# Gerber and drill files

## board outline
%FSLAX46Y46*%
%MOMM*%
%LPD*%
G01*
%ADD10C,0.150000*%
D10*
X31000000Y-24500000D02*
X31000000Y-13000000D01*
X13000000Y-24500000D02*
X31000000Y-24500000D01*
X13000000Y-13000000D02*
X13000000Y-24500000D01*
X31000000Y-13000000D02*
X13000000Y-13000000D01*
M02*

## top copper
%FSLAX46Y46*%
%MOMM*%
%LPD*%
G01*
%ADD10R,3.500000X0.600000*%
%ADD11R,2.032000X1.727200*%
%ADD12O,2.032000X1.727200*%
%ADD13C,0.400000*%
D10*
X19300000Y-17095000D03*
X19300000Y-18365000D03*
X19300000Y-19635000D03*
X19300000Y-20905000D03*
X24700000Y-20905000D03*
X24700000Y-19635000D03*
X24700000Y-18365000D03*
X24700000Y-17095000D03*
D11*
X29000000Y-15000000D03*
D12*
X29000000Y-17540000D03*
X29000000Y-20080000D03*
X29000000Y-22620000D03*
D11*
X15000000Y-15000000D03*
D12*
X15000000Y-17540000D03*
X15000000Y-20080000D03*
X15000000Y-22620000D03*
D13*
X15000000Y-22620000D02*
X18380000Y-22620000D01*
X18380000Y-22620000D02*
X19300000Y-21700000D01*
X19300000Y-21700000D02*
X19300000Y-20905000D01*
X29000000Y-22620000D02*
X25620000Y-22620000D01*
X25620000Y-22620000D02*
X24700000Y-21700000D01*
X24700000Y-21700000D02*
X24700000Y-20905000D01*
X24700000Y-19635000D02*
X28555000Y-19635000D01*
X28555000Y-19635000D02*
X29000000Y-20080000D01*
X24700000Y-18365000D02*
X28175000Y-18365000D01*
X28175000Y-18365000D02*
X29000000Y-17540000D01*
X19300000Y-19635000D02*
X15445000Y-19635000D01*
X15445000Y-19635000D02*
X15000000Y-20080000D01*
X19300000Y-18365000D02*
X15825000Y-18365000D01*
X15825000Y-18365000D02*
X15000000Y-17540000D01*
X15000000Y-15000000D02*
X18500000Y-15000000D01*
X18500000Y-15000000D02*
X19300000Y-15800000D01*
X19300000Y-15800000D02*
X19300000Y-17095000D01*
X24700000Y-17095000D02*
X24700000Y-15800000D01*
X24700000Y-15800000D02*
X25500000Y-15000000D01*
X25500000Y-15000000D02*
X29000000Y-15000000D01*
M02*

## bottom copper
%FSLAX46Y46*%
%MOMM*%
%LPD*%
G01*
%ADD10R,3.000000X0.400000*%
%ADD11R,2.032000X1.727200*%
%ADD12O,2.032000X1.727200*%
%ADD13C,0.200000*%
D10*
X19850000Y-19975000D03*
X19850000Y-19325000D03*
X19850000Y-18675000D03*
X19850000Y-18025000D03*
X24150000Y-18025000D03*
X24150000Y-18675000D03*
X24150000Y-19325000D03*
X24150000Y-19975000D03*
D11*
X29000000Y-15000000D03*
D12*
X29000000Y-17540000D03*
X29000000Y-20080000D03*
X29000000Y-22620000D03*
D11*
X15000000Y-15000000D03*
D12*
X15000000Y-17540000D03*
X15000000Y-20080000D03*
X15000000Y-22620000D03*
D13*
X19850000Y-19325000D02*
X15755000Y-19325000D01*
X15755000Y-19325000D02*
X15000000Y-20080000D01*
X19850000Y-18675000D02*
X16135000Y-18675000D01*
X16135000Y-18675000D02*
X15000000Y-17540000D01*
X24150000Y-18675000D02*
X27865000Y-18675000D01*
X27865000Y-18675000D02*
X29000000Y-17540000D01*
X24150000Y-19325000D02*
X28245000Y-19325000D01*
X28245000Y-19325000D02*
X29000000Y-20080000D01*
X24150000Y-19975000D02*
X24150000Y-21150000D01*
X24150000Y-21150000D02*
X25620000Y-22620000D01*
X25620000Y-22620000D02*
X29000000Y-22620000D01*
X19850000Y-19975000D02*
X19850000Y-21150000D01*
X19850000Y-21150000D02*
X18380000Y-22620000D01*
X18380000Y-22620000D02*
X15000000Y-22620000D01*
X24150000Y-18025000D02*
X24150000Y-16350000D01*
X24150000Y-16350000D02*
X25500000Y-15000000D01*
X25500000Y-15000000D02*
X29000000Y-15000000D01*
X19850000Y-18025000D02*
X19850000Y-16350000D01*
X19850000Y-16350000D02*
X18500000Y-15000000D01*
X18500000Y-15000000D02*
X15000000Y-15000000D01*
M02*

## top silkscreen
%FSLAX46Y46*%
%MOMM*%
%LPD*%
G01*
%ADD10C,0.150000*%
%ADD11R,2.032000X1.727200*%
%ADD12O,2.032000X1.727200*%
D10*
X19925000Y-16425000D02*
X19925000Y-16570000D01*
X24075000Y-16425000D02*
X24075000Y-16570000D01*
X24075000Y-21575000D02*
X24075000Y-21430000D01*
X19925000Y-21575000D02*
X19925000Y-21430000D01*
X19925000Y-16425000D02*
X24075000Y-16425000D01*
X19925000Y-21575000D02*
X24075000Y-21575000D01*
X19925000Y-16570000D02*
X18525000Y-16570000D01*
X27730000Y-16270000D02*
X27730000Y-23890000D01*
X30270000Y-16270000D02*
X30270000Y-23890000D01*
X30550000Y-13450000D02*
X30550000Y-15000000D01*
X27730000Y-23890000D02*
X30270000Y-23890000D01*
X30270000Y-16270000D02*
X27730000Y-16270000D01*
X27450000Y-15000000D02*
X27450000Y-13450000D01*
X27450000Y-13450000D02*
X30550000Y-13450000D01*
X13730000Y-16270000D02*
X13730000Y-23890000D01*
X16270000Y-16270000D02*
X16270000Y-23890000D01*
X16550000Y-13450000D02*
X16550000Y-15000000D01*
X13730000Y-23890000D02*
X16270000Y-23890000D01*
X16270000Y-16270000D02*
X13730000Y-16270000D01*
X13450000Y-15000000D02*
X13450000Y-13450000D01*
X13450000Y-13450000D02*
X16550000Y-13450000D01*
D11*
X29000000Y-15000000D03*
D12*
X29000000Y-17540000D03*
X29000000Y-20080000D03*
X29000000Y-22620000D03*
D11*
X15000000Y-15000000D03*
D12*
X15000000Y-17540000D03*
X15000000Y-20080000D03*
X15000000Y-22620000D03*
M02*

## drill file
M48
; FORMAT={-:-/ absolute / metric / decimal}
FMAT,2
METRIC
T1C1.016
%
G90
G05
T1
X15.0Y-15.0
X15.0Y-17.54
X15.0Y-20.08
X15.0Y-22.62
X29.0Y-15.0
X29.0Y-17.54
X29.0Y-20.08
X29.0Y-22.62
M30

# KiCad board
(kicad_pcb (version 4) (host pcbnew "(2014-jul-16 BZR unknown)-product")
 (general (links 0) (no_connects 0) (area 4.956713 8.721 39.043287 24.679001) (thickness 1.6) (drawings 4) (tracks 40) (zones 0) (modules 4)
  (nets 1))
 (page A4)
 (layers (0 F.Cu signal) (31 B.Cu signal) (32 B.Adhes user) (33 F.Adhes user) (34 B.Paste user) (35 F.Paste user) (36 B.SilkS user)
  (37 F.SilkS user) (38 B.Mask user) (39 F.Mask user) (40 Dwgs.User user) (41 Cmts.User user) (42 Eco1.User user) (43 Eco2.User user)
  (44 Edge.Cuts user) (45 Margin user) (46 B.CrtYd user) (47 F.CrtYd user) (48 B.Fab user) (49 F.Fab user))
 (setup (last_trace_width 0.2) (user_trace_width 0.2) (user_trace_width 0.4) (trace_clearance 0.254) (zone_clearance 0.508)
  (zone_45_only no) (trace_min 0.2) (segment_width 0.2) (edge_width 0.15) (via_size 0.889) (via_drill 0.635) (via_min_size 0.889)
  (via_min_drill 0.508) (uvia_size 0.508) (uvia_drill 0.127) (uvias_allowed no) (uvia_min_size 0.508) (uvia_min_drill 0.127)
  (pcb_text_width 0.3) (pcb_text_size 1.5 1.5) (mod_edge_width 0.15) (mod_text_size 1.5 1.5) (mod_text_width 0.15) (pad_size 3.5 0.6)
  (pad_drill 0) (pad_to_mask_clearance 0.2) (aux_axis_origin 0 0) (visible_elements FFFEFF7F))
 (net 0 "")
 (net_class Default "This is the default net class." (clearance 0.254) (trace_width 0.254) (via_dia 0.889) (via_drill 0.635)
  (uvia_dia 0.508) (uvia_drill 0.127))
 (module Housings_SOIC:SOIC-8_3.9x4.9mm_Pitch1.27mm (layer F.Cu) (at 22 19)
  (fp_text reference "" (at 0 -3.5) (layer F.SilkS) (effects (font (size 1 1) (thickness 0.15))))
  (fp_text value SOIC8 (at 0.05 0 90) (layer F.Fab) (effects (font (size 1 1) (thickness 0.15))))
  (fp_line (start -2.075 -2.575) (end -2.075 -2.43) (layer F.SilkS) (width 0.15))
  (fp_line (start 2.075 -2.575) (end 2.075 -2.43) (layer F.SilkS) (width 0.15))
  (fp_line (start 2.075 2.575) (end 2.075 2.43) (layer F.SilkS) (width 0.15))
  (fp_line (start -2.075 2.575) (end -2.075 2.43) (layer F.SilkS) (width 0.15))
  (fp_line (start -2.075 -2.575) (end 2.075 -2.575) (layer F.SilkS) (width 0.15))
  (fp_line (start -2.075 2.575) (end 2.075 2.575) (layer F.SilkS) (width 0.15))
  (fp_line (start -2.075 -2.43) (end -3.475 -2.43) (layer F.SilkS) (width 0.15))
  (pad 1 smd rect (at -2.7 -1.905) (size 3.5 0.6) (layers F.Cu F.Paste F.Mask))
  (pad 2 smd rect (at -2.7 -0.635) (size 3.5 0.6) (layers F.Cu F.Paste F.Mask))
  (pad 3 smd rect (at -2.7 0.635) (size 3.5 0.6) (layers F.Cu F.Paste F.Mask))
  (pad 4 smd rect (at -2.7 1.905) (size 3.5 0.6) (layers F.Cu F.Paste F.Mask))
  (pad 5 smd rect (at 2.7 1.905) (size 3.5 0.6) (layers F.Cu F.Paste F.Mask))
  (pad 6 smd rect (at 2.7 0.635) (size 3.5 0.6) (layers F.Cu F.Paste F.Mask))
  (pad 7 smd rect (at 2.7 -0.635) (size 3.5 0.6) (layers F.Cu F.Paste F.Mask))
  (pad 8 smd rect (at 2.7 -1.905) (size 3.5 0.6) (layers F.Cu F.Paste F.Mask)))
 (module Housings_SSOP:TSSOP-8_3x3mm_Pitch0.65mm (layer B.Cu) (at 22 19)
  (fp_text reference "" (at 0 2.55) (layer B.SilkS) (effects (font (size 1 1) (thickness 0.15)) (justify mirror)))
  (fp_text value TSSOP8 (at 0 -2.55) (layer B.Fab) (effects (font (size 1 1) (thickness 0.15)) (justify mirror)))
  (pad 1 smd rect (at -2.15 0.975) (size 3 0.4) (layers B.Cu B.Paste B.Mask))
  (pad 2 smd rect (at -2.15 0.325) (size 3 0.4) (layers B.Cu B.Paste B.Mask))
  (pad 3 smd rect (at -2.15 -0.325) (size 3 0.4) (layers B.Cu B.Paste B.Mask))
  (pad 4 smd rect (at -2.15 -0.975) (size 3 0.4) (layers B.Cu B.Paste B.Mask))
  (pad 5 smd rect (at 2.15 -0.975) (size 3 0.4) (layers B.Cu B.Paste B.Mask))
  (pad 6 smd rect (at 2.15 -0.325) (size 3 0.4) (layers B.Cu B.Paste B.Mask))
  (pad 7 smd rect (at 2.15 0.325) (size 3 0.4) (layers B.Cu B.Paste B.Mask))
  (pad 8 smd rect (at 2.15 0.975) (size 3 0.4) (layers B.Cu B.Paste B.Mask)))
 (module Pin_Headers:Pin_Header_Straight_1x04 (layer F.Cu) (at 29 15)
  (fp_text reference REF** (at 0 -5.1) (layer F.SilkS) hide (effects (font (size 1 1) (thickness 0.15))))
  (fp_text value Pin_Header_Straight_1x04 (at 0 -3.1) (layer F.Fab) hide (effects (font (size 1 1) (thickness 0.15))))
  (fp_line (start -1.27 1.27) (end -1.27 8.89) (layer F.SilkS) (width 0.15))
  (fp_line (start 1.27 1.27) (end 1.27 8.89) (layer F.SilkS) (width 0.15))
  (fp_line (start 1.55 -1.55) (end 1.55 0) (layer F.SilkS) (width 0.15))
  (fp_line (start -1.27 8.89) (end 1.27 8.89) (layer F.SilkS) (width 0.15))
  (fp_line (start 1.27 1.27) (end -1.27 1.27) (layer F.SilkS) (width 0.15))
  (fp_line (start -1.55 0) (end -1.55 -1.55) (layer F.SilkS) (width 0.15))
  (fp_line (start -1.55 -1.55) (end 1.55 -1.55) (layer F.SilkS) (width 0.15))
  (pad 1 thru_hole rect (at 0 0) (size 2.032 1.7272) (drill 1.016) (layers *.Cu *.Mask F.SilkS))
  (pad 2 thru_hole oval (at 0 2.54) (size 2.032 1.7272) (drill 1.016) (layers *.Cu *.Mask F.SilkS))
  (pad 3 thru_hole oval (at 0 5.08) (size 2.032 1.7272) (drill 1.016) (layers *.Cu *.Mask F.SilkS))
  (pad 4 thru_hole oval (at 0 7.62) (size 2.032 1.7272) (drill 1.016) (layers *.Cu *.Mask F.SilkS)))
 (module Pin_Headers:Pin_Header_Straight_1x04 (layer F.Cu) (at 15 15)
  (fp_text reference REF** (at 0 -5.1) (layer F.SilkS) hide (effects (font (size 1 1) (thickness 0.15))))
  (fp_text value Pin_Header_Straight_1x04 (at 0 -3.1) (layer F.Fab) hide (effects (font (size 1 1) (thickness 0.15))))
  (fp_line (start -1.27 1.27) (end -1.27 8.89) (layer F.SilkS) (width 0.15))
  (fp_line (start 1.27 1.27) (end 1.27 8.89) (layer F.SilkS) (width 0.15))
  (fp_line (start 1.55 -1.55) (end 1.55 0) (layer F.SilkS) (width 0.15))
  (fp_line (start -1.27 8.89) (end 1.27 8.89) (layer F.SilkS) (width 0.15))
  (fp_line (start 1.27 1.27) (end -1.27 1.27) (layer F.SilkS) (width 0.15))
  (fp_line (start -1.55 0) (end -1.55 -1.55) (layer F.SilkS) (width 0.15))
  (fp_line (start -1.55 -1.55) (end 1.55 -1.55) (layer F.SilkS) (width 0.15))
  (pad 1 thru_hole rect (at 0 0) (size 2.032 1.7272) (drill 1.016) (layers *.Cu *.Mask F.SilkS))
  (pad 2 thru_hole oval (at 0 2.54) (size 2.032 1.7272) (drill 1.016) (layers *.Cu *.Mask F.SilkS))
  (pad 3 thru_hole oval (at 0 5.08) (size 2.032 1.7272) (drill 1.016) (layers *.Cu *.Mask F.SilkS))
  (pad 4 thru_hole oval (at 0 7.62) (size 2.032 1.7272) (drill 1.016) (layers *.Cu *.Mask F.SilkS)))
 (gr_line (start 31 24.5) (end 31 13) (angle 90) (layer Edge.Cuts) (width 0.15))
 (gr_line (start 13 24.5) (end 31 24.5) (angle 90) (layer Edge.Cuts) (width 0.15))
 (gr_line (start 13 13) (end 13 24.5) (angle 90) (layer Edge.Cuts) (width 0.15))
 (gr_line (start 31 13) (end 13 13) (angle 90) (layer Edge.Cuts) (width 0.15))
 (segment (start 19.85 19.325) (end 15.755 19.325) (width 0.2) (layer B.Cu) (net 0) (status 400000))
 (segment (start 15.755 19.325) (end 15 20.08) (width 0.2) (layer B.Cu) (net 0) (status 800000))
 (segment (start 19.85 18.675) (end 16.135 18.675) (width 0.2) (layer B.Cu) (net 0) (status 400000))
 (segment (start 16.135 18.675) (end 15 17.54) (width 0.2) (layer B.Cu) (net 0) (status 800000))
 (segment (start 24.15 18.675) (end 27.865 18.675) (width 0.2) (layer B.Cu) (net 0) (status 400000))
 (segment (start 27.865 18.675) (end 29 17.54) (width 0.2) (layer B.Cu) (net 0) (status 800000))
 (segment (start 24.15 19.325) (end 28.245 19.325) (width 0.2) (layer B.Cu) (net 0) (status 400000))
 (segment (start 28.245 19.325) (end 29 20.08) (width 0.2) (layer B.Cu) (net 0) (status 800000))
 (segment (start 24.15 19.975) (end 24.15 21.15) (width 0.2) (layer B.Cu) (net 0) (status 400000))
 (segment (start 24.15 21.15) (end 25.62 22.62) (width 0.2) (layer B.Cu) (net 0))
 (segment (start 25.62 22.62) (end 29 22.62) (width 0.2) (layer B.Cu) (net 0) (status 800000))
 (segment (start 19.85 19.975) (end 19.85 21.15) (width 0.2) (layer B.Cu) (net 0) (status 400000))
 (segment (start 19.85 21.15) (end 18.38 22.62) (width 0.2) (layer B.Cu) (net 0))
 (segment (start 18.38 22.62) (end 15 22.62) (width 0.2) (layer B.Cu) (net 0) (status 800000))
 (segment (start 24.15 18.025) (end 24.15 16.35) (width 0.2) (layer B.Cu) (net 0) (status 400000))
 (segment (start 24.15 16.35) (end 25.5 15) (width 0.2) (layer B.Cu) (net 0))
 (segment (start 25.5 15) (end 29 15) (width 0.2) (layer B.Cu) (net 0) (status 800000))
 (segment (start 19.85 18.025) (end 19.85 16.35) (width 0.2) (layer B.Cu) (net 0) (status 400000))
 (segment (start 19.85 16.35) (end 18.5 15) (width 0.2) (layer B.Cu) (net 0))
 (segment (start 18.5 15) (end 15 15) (width 0.2) (layer B.Cu) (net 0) (status 800000))
 (segment (start 15 22.62) (end 18.38 22.62) (width 0.4) (layer F.Cu) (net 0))
 (segment (start 18.38 22.62) (end 19.3 21.7) (width 0.4) (layer F.Cu) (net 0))
 (segment (start 19.3 21.7) (end 19.3 20.905) (width 0.4) (layer F.Cu) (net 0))
 (segment (start 29 22.62) (end 25.62 22.62) (width 0.4) (layer F.Cu) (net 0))
 (segment (start 25.62 22.62) (end 24.7 21.7) (width 0.4) (layer F.Cu) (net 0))
 (segment (start 24.7 21.7) (end 24.7 20.905) (width 0.4) (layer F.Cu) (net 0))
 (segment (start 24.7 19.635) (end 28.555 19.635) (width 0.4) (layer F.Cu) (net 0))
 (segment (start 28.555 19.635) (end 29 20.08) (width 0.4) (layer F.Cu) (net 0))
 (segment (start 24.7 18.365) (end 28.175 18.365) (width 0.4) (layer F.Cu) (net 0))
 (segment (start 28.175 18.365) (end 29 17.54) (width 0.4) (layer F.Cu) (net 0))
 (segment (start 19.3 19.635) (end 15.445 19.635) (width 0.4) (layer F.Cu) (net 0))
 (segment (start 15.445 19.635) (end 15 20.08) (width 0.4) (layer F.Cu) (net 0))
 (segment (start 19.3 18.365) (end 15.825 18.365) (width 0.4) (layer F.Cu) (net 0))
 (segment (start 15.825 18.365) (end 15 17.54) (width 0.4) (layer F.Cu) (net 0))
 (segment (start 15 15) (end 18.5 15) (width 0.4) (layer F.Cu) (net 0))
 (segment (start 18.5 15) (end 19.3 15.8) (width 0.4) (layer F.Cu) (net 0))
 (segment (start 19.3 15.8) (end 19.3 17.095) (width 0.4) (layer F.Cu) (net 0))
 (segment (start 24.7 17.095) (end 24.7 15.8) (width 0.4) (layer F.Cu) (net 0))
 (segment (start 24.7 15.8) (end 25.5 15) (width 0.4) (layer F.Cu) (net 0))
 (segment (start 25.5 15) (end 29 15) (width 0.4) (layer F.Cu) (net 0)))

